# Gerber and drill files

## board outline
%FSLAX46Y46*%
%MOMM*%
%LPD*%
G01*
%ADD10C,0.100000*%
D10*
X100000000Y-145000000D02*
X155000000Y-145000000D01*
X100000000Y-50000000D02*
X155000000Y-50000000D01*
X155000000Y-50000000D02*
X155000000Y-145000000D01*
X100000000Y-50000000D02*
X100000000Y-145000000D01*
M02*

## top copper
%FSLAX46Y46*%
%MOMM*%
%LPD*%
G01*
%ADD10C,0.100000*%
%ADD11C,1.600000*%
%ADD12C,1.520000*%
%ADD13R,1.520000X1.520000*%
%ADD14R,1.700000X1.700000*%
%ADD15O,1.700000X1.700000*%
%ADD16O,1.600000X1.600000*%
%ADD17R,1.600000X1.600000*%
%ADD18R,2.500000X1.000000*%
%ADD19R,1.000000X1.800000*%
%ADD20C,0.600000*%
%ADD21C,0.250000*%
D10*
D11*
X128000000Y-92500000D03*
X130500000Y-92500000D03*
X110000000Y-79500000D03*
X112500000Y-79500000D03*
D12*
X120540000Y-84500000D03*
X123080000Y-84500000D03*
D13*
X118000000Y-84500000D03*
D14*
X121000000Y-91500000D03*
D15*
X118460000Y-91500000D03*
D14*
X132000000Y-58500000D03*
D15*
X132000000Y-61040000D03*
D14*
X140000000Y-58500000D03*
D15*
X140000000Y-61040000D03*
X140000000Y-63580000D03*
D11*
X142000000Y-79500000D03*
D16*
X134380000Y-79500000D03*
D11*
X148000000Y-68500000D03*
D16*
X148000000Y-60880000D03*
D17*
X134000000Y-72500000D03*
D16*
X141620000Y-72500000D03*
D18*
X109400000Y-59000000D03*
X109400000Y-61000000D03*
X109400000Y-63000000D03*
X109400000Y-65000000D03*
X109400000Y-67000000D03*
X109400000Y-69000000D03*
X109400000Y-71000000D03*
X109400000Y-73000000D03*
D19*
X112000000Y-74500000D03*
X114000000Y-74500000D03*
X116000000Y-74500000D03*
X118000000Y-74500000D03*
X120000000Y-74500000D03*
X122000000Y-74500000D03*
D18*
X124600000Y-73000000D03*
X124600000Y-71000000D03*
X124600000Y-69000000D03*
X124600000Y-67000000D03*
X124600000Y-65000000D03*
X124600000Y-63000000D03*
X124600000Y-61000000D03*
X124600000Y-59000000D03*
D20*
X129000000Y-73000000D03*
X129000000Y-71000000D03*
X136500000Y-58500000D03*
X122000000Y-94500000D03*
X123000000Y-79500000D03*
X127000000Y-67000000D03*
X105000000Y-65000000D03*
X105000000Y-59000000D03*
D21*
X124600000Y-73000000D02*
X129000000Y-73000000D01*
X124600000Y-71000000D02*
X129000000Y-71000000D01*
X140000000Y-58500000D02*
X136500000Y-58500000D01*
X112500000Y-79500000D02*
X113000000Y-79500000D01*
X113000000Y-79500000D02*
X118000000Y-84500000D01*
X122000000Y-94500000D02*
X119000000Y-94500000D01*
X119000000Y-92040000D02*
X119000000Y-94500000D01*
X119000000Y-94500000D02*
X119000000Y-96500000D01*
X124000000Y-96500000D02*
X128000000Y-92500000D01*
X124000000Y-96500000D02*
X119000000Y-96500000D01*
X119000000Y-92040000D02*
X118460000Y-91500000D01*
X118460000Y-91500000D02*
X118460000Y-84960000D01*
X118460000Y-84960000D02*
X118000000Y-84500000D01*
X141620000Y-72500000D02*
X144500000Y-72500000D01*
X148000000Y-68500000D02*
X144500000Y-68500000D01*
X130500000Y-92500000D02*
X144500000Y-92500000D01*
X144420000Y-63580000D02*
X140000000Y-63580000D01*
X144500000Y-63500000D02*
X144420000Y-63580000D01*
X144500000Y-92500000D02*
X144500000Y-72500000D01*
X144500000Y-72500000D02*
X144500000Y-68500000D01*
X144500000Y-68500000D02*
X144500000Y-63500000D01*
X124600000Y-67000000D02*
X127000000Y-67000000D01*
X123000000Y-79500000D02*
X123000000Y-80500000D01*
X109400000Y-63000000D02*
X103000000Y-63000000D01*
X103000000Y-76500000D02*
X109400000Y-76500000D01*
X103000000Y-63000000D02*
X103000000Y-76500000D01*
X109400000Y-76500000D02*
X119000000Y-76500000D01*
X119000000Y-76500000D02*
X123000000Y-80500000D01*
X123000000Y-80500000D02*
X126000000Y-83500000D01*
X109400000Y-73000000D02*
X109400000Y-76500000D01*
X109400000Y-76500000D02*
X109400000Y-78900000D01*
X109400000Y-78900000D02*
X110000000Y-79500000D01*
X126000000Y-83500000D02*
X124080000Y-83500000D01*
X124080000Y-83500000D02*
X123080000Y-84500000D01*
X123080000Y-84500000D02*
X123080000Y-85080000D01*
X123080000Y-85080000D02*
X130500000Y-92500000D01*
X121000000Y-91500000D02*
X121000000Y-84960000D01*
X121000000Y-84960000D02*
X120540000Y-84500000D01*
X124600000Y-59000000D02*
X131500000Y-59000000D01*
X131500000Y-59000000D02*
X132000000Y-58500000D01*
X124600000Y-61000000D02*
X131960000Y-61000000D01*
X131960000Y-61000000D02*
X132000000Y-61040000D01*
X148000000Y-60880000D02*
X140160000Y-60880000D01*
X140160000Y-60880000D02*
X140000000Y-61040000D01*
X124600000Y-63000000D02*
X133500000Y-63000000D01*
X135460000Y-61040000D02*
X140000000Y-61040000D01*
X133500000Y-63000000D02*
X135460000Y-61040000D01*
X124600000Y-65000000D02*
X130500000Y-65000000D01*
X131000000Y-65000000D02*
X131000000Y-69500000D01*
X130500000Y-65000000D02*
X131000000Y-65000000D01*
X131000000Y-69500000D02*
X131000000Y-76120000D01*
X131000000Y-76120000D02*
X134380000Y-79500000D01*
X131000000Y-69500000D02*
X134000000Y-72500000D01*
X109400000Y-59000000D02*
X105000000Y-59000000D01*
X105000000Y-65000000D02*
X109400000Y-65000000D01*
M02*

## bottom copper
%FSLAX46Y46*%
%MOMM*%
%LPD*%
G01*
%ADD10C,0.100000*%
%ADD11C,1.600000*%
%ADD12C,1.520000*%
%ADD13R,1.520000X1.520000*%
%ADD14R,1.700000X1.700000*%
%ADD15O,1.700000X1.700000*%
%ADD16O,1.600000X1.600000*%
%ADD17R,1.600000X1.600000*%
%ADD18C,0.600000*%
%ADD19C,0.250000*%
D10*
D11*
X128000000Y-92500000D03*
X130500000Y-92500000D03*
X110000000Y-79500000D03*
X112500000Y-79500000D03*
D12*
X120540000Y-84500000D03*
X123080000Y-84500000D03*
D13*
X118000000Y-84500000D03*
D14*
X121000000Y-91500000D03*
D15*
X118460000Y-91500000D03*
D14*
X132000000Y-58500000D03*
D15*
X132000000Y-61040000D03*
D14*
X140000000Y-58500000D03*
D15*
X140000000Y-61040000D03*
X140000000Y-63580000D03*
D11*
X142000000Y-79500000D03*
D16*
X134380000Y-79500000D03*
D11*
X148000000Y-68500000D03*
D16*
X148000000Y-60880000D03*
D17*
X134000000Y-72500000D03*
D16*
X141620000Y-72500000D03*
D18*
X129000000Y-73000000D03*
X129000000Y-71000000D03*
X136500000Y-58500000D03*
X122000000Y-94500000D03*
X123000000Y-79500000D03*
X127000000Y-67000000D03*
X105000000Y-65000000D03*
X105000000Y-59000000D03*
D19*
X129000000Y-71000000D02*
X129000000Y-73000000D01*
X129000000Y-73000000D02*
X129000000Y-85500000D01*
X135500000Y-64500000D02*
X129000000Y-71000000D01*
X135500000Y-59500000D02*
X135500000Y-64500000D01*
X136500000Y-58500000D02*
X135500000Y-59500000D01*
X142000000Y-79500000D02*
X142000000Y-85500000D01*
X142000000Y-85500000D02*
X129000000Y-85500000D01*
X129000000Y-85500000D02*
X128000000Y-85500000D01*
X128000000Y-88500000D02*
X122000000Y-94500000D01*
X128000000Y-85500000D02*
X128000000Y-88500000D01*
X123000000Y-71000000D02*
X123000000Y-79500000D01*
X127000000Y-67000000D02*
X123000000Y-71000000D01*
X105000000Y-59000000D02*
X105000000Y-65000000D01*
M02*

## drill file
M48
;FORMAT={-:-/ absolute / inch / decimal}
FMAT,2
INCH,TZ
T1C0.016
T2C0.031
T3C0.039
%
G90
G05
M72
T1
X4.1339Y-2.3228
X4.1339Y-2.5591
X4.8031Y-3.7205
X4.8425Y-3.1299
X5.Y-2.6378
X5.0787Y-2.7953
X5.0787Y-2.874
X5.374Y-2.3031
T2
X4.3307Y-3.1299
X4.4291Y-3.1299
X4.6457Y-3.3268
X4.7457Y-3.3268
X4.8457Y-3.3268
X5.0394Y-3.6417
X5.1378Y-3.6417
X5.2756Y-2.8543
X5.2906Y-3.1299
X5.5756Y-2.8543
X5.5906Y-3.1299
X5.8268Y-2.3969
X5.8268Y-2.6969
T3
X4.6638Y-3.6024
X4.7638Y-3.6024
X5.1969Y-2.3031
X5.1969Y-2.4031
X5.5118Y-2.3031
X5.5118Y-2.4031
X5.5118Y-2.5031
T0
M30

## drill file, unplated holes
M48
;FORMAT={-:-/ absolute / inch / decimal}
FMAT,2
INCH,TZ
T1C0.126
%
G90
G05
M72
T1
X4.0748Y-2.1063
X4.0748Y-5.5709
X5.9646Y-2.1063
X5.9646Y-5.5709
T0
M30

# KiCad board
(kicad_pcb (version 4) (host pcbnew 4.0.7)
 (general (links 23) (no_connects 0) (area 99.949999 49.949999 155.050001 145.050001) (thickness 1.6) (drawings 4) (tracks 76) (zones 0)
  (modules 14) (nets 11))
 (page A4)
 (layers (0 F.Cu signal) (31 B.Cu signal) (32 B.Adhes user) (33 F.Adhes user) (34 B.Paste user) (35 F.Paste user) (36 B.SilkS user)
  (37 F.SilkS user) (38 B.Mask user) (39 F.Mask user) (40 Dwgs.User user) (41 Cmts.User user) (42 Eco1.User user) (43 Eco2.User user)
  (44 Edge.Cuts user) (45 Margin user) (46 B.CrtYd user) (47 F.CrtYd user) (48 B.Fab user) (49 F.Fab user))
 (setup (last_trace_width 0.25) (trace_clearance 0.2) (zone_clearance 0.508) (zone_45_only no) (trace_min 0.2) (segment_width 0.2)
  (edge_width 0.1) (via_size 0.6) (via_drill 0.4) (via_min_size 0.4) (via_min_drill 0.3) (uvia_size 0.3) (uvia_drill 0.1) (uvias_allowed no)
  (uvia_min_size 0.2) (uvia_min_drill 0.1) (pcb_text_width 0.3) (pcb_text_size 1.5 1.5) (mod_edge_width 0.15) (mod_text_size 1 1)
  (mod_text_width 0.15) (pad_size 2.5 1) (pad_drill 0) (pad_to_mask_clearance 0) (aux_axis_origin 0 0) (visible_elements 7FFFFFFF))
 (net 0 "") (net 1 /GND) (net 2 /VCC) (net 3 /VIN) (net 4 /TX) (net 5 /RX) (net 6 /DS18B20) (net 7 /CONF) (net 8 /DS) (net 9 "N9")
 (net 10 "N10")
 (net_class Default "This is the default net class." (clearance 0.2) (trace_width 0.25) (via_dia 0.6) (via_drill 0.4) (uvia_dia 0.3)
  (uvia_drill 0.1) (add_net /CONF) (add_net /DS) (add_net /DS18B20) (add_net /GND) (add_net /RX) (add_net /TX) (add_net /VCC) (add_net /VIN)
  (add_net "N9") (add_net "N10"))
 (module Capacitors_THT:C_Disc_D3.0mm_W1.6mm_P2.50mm (layer F.Cu) (at 128 92.5)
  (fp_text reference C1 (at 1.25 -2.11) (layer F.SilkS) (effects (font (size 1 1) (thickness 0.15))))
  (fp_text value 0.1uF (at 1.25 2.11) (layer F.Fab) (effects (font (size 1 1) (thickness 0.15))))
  (pad 1 thru_hole circle (at 0 0) (size 1.6 1.6) (drill 0.8) (layers *.Cu *.Mask) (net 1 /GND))
  (pad 2 thru_hole circle (at 2.5 0) (size 1.6 1.6) (drill 0.8) (layers *.Cu *.Mask) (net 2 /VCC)))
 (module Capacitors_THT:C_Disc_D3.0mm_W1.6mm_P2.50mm (layer F.Cu) (at 110 79.5)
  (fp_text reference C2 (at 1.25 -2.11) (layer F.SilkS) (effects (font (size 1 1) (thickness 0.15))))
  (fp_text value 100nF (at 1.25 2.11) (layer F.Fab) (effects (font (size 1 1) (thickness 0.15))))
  (pad 1 thru_hole circle (at 0 0) (size 1.6 1.6) (drill 0.8) (layers *.Cu *.Mask) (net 2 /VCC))
  (pad 2 thru_hole circle (at 2.5 0) (size 1.6 1.6) (drill 0.8) (layers *.Cu *.Mask) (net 1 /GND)))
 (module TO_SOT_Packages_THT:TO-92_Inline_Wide (layer F.Cu) (at 118 84.5)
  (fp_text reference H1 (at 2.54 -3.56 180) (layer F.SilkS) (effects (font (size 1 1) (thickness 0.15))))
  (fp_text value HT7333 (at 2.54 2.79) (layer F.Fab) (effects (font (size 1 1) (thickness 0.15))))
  (pad 2 thru_hole circle (at 2.54 0 90) (size 1.52 1.52) (drill 0.8) (layers *.Cu *.Mask) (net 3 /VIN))
  (pad 3 thru_hole circle (at 5.08 0 90) (size 1.52 1.52) (drill 0.8) (layers *.Cu *.Mask) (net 2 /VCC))
  (pad 1 thru_hole rect (at 0 0 90) (size 1.52 1.52) (drill 0.8) (layers *.Cu *.Mask) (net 1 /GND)))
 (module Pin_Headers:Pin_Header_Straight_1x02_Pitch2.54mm (layer F.Cu) (at 121 91.5 270)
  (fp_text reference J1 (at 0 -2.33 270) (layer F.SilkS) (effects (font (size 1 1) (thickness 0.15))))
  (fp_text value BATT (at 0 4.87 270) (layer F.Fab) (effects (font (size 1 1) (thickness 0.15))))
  (pad 1 thru_hole rect (at 0 0 270) (size 1.7 1.7) (drill 1) (layers *.Cu *.Mask) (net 3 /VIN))
  (pad 2 thru_hole oval (at 0 2.54 270) (size 1.7 1.7) (drill 1) (layers *.Cu *.Mask) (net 1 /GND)))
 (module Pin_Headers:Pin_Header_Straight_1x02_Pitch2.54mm (layer F.Cu) (at 132 58.5)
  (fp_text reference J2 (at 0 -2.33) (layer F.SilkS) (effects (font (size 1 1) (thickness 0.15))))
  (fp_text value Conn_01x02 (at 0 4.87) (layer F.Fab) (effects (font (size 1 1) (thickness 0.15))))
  (pad 1 thru_hole rect (at 0 0) (size 1.7 1.7) (drill 1) (layers *.Cu *.Mask) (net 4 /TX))
  (pad 2 thru_hole oval (at 0 2.54) (size 1.7 1.7) (drill 1) (layers *.Cu *.Mask) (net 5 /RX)))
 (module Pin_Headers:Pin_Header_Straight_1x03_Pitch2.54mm (layer F.Cu) (at 140 58.5)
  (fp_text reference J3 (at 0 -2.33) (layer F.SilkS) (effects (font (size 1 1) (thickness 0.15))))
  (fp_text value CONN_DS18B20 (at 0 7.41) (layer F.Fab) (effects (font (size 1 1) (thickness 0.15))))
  (pad 1 thru_hole rect (at 0 0) (size 1.7 1.7) (drill 1) (layers *.Cu *.Mask) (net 1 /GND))
  (pad 2 thru_hole oval (at 0 2.54) (size 1.7 1.7) (drill 1) (layers *.Cu *.Mask) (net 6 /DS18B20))
  (pad 3 thru_hole oval (at 0 5.08) (size 1.7 1.7) (drill 1) (layers *.Cu *.Mask) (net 2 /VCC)))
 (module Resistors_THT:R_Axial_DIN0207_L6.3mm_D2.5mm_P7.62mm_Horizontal (layer F.Cu) (at 142 79.5 180)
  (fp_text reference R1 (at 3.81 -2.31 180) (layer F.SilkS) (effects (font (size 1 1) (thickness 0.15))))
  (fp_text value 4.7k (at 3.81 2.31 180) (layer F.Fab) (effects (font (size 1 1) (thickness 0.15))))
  (pad 1 thru_hole circle (at 0 0 180) (size 1.6 1.6) (drill 0.8) (layers *.Cu *.Mask) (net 1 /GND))
  (pad 2 thru_hole oval (at 7.62 0 180) (size 1.6 1.6) (drill 0.8) (layers *.Cu *.Mask) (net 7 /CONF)))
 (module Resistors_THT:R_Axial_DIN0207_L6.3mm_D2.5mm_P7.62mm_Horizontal (layer F.Cu) (at 148 68.5 90)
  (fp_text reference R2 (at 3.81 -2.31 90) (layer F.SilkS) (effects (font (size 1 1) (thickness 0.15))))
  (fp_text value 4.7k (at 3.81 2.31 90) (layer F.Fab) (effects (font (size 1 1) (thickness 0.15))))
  (pad 1 thru_hole circle (at 0 0 90) (size 1.6 1.6) (drill 0.8) (layers *.Cu *.Mask) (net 2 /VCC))
  (pad 2 thru_hole oval (at 7.62 0 90) (size 1.6 1.6) (drill 0.8) (layers *.Cu *.Mask) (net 6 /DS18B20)))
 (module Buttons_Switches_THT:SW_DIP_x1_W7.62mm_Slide (layer F.Cu) (at 134 72.5)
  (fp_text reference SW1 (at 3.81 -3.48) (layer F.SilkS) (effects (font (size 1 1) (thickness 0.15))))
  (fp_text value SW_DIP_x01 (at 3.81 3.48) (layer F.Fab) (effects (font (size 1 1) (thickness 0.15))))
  (pad 1 thru_hole rect (at 0 0) (size 1.6 1.6) (drill 0.8) (layers *.Cu *.Mask) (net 7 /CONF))
  (pad 2 thru_hole oval (at 7.62 0) (size 1.6 1.6) (drill 0.8) (layers *.Cu *.Mask) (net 2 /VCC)))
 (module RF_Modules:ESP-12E (layer F.Cu) (at 117 62.5)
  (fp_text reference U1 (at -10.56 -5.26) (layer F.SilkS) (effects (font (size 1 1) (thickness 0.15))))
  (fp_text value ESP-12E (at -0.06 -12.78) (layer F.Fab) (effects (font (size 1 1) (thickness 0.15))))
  (pad 1 smd rect (at -7.6 -3.5) (size 2.5 1) (layers F.Cu F.Paste F.Mask) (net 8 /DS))
  (pad 2 smd rect (at -7.6 -1.5) (size 2.5 1) (layers F.Cu F.Paste F.Mask))
  (pad 3 smd rect (at -7.6 0.5) (size 2.5 1) (layers F.Cu F.Paste F.Mask) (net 2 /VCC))
  (pad 4 smd rect (at -7.6 2.5) (size 2.5 1) (layers F.Cu F.Paste F.Mask) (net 8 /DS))
  (pad 5 smd rect (at -7.6 4.5) (size 2.5 1) (layers F.Cu F.Paste F.Mask))
  (pad 6 smd rect (at -7.6 6.5) (size 2.5 1) (layers F.Cu F.Paste F.Mask))
  (pad 7 smd rect (at -7.6 8.5) (size 2.5 1) (layers F.Cu F.Paste F.Mask))
  (pad 8 smd rect (at -7.6 10.5) (size 2.5 1) (layers F.Cu F.Paste F.Mask) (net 2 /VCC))
  (pad 9 smd rect (at -5 12) (size 1 1.8) (layers F.Cu F.Paste F.Mask))
  (pad 10 smd rect (at -3 12) (size 1 1.8) (layers F.Cu F.Paste F.Mask))
  (pad 11 smd rect (at -1 12) (size 1 1.8) (layers F.Cu F.Paste F.Mask) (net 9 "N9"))
  (pad 12 smd rect (at 1 12) (size 1 1.8) (layers F.Cu F.Paste F.Mask) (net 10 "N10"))
  (pad 13 smd rect (at 3 12) (size 1 1.8) (layers F.Cu F.Paste F.Mask))
  (pad 14 smd rect (at 5 12) (size 1 1.8) (layers F.Cu F.Paste F.Mask))
  (pad 15 smd rect (at 7.6 10.5) (size 2.5 1) (layers F.Cu F.Paste F.Mask) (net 1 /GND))
  (pad 16 smd rect (at 7.6 8.5) (size 2.5 1) (layers F.Cu F.Paste F.Mask) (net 1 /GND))
  (pad 17 smd rect (at 7.6 6.5) (size 2.5 1) (layers F.Cu F.Paste F.Mask))
  (pad 18 smd rect (at 7.6 4.5) (size 2.5 1) (layers F.Cu F.Paste F.Mask) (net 2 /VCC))
  (pad 19 smd rect (at 7.6 2.5) (size 2.5 1) (layers F.Cu F.Paste F.Mask) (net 7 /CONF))
  (pad 20 smd rect (at 7.6 0.5) (size 2.5 1) (layers F.Cu F.Paste F.Mask) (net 6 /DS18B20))
  (pad 21 smd rect (at 7.6 -1.5) (size 2.5 1) (layers F.Cu F.Paste F.Mask) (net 5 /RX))
  (pad 22 smd rect (at 7.6 -3.5) (size 2.5 1) (layers F.Cu F.Paste F.Mask) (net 4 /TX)))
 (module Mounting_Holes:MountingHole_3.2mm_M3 (layer F.Cu) (at 103.5 53.5)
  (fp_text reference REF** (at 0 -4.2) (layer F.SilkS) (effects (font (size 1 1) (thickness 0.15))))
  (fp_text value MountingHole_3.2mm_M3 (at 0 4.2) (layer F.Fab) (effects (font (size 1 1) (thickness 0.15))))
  (pad 1 np_thru_hole circle (at 0 0) (size 3.2 3.2) (drill 3.2) (layers *.Cu *.Mask)))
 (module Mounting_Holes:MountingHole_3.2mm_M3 (layer F.Cu) (at 151.5 53.5)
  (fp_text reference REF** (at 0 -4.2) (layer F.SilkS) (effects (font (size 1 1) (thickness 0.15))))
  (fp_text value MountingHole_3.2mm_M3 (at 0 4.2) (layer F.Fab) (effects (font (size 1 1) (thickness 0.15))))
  (pad 1 np_thru_hole circle (at 0 0) (size 3.2 3.2) (drill 3.2) (layers *.Cu *.Mask)))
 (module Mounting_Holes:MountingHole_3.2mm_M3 (layer F.Cu) (at 151.5 141.5)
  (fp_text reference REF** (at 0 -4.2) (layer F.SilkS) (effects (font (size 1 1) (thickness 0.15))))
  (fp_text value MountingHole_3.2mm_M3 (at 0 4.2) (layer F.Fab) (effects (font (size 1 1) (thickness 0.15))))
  (pad 1 np_thru_hole circle (at 0 0) (size 3.2 3.2) (drill 3.2) (layers *.Cu *.Mask)))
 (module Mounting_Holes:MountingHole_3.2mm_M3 (layer F.Cu) (at 103.5 141.5)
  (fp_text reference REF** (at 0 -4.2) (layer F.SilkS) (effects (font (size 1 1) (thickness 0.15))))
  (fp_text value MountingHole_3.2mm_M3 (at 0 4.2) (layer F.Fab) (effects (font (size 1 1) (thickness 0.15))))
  (pad 1 np_thru_hole circle (at 0 0) (size 3.2 3.2) (drill 3.2) (layers *.Cu *.Mask)))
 (gr_line (start 100 145) (end 155 145) (angle 90) (layer Edge.Cuts) (width 0.1))
 (gr_line (start 100 50) (end 155 50) (angle 90) (layer Edge.Cuts) (width 0.1))
 (gr_line (start 155 50) (end 155 145) (angle 90) (layer Edge.Cuts) (width 0.1))
 (gr_line (start 100 50) (end 100 145) (angle 90) (layer Edge.Cuts) (width 0.1))
 (segment (start 124.6 73) (end 129 73) (width 0.25) (layer F.Cu) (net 1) (status 400000))
 (via (at 129 73) (size 0.6) (drill 0.4) (layers F.Cu B.Cu) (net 1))
 (segment (start 124.6 71) (end 129 71) (width 0.25) (layer F.Cu) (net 1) (status 400000))
 (via (at 129 71) (size 0.6) (drill 0.4) (layers F.Cu B.Cu) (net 1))
 (segment (start 140 58.5) (end 136.5 58.5) (width 0.25) (layer F.Cu) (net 1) (status 400000))
 (segment (start 129 71) (end 129 73) (width 0.25) (layer B.Cu) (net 1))
 (segment (start 129 73) (end 129 85.5) (width 0.25) (layer B.Cu) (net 1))
 (segment (start 135.5 64.5) (end 129 71) (width 0.25) (layer B.Cu) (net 1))
 (segment (start 135.5 59.5) (end 135.5 64.5) (width 0.25) (layer B.Cu) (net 1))
 (segment (start 136.5 58.5) (end 135.5 59.5) (width 0.25) (layer B.Cu) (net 1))
 (via (at 136.5 58.5) (size 0.6) (drill 0.4) (layers F.Cu B.Cu) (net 1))
 (segment (start 142 79.5) (end 142 85.5) (width 0.25) (layer B.Cu) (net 1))
 (segment (start 142 85.5) (end 129 85.5) (width 0.25) (layer B.Cu) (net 1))
 (segment (start 129 85.5) (end 128 85.5) (width 0.25) (layer B.Cu) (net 1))
 (segment (start 112.5 79.5) (end 113 79.5) (width 0.25) (layer F.Cu) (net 1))
 (segment (start 113 79.5) (end 118 84.5) (width 0.25) (layer F.Cu) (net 1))
 (segment (start 128 88.5) (end 122 94.5) (width 0.25) (layer B.Cu) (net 1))
 (segment (start 128 85.5) (end 128 88.5) (width 0.25) (layer B.Cu) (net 1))
 (segment (start 122 94.5) (end 119 94.5) (width 0.25) (layer F.Cu) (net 1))
 (via (at 122 94.5) (size 0.6) (drill 0.4) (layers F.Cu B.Cu) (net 1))
 (segment (start 119 92.04) (end 119 94.5) (width 0.25) (layer F.Cu) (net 1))
 (segment (start 119 94.5) (end 119 96.5) (width 0.25) (layer F.Cu) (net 1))
 (segment (start 124 96.5) (end 128 92.5) (width 0.25) (layer F.Cu) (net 1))
 (segment (start 124 96.5) (end 119 96.5) (width 0.25) (layer F.Cu) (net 1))
 (segment (start 119 92.04) (end 118.46 91.5) (width 0.25) (layer F.Cu) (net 1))
 (segment (start 118.46 91.5) (end 118.46 84.96) (width 0.25) (layer F.Cu) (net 1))
 (segment (start 118.46 84.96) (end 118 84.5) (width 0.25) (layer F.Cu) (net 1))
 (segment (start 141.62 72.5) (end 144.5 72.5) (width 0.25) (layer F.Cu) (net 2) (status 400000))
 (segment (start 148 68.5) (end 144.5 68.5) (width 0.25) (layer F.Cu) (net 2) (status 400000))
 (segment (start 130.5 92.5) (end 144.5 92.5) (width 0.25) (layer F.Cu) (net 2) (status 400000))
 (segment (start 144.42 63.58) (end 140 63.58) (width 0.25) (layer F.Cu) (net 2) (status 800000))
 (segment (start 144.5 63.5) (end 144.42 63.58) (width 0.25) (layer F.Cu) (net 2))
 (segment (start 144.5 92.5) (end 144.5 72.5) (width 0.25) (layer F.Cu) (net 2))
 (segment (start 144.5 72.5) (end 144.5 68.5) (width 0.25) (layer F.Cu) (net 2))
 (segment (start 144.5 68.5) (end 144.5 63.5) (width 0.25) (layer F.Cu) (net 2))
 (segment (start 124.6 67) (end 127 67) (width 0.25) (layer F.Cu) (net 2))
 (segment (start 123 79.5) (end 123 80.5) (width 0.25) (layer F.Cu) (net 2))
 (via (at 123 79.5) (size 0.6) (drill 0.4) (layers F.Cu B.Cu) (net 2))
 (segment (start 123 71) (end 123 79.5) (width 0.25) (layer B.Cu) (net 2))
 (segment (start 127 67) (end 123 71) (width 0.25) (layer B.Cu) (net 2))
 (via (at 127 67) (size 0.6) (drill 0.4) (layers F.Cu B.Cu) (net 2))
 (segment (start 109.4 63) (end 103 63) (width 0.25) (layer F.Cu) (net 2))
 (segment (start 103 76.5) (end 109.4 76.5) (width 0.25) (layer F.Cu) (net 2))
 (segment (start 103 63) (end 103 76.5) (width 0.25) (layer F.Cu) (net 2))
 (segment (start 109.4 76.5) (end 119 76.5) (width 0.25) (layer F.Cu) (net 2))
 (segment (start 119 76.5) (end 123 80.5) (width 0.25) (layer F.Cu) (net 2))
 (segment (start 123 80.5) (end 126 83.5) (width 0.25) (layer F.Cu) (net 2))
 (segment (start 109.4 73) (end 109.4 76.5) (width 0.25) (layer F.Cu) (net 2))
 (segment (start 109.4 76.5) (end 109.4 78.9) (width 0.25) (layer F.Cu) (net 2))
 (segment (start 109.4 78.9) (end 110 79.5) (width 0.25) (layer F.Cu) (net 2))
 (segment (start 126 83.5) (end 124.08 83.5) (width 0.25) (layer F.Cu) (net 2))
 (segment (start 124.08 83.5) (end 123.08 84.5) (width 0.25) (layer F.Cu) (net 2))
 (segment (start 123.08 84.5) (end 123.08 85.08) (width 0.25) (layer F.Cu) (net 2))
 (segment (start 123.08 85.08) (end 130.5 92.5) (width 0.25) (layer F.Cu) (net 2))
 (segment (start 121 91.5) (end 121 84.96) (width 0.25) (layer F.Cu) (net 3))
 (segment (start 121 84.96) (end 120.54 84.5) (width 0.25) (layer F.Cu) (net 3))
 (segment (start 124.6 59) (end 131.5 59) (width 0.25) (layer F.Cu) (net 4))
 (segment (start 131.5 59) (end 132 58.5) (width 0.25) (layer F.Cu) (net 4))
 (segment (start 124.6 61) (end 131.96 61) (width 0.25) (layer F.Cu) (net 5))
 (segment (start 131.96 61) (end 132 61.04) (width 0.25) (layer F.Cu) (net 5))
 (segment (start 148 60.88) (end 140.16 60.88) (width 0.25) (layer F.Cu) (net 6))
 (segment (start 140.16 60.88) (end 140 61.04) (width 0.25) (layer F.Cu) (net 6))
 (segment (start 124.6 63) (end 133.5 63) (width 0.25) (layer F.Cu) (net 6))
 (segment (start 135.46 61.04) (end 140 61.04) (width 0.25) (layer F.Cu) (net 6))
 (segment (start 133.5 63) (end 135.46 61.04) (width 0.25) (layer F.Cu) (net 6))
 (segment (start 124.6 65) (end 130.5 65) (width 0.25) (layer F.Cu) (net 7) (status 400000))
 (segment (start 131 65) (end 131 69.5) (width 0.25) (layer F.Cu) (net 7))
 (segment (start 130.5 65) (end 131 65) (width 0.25) (layer F.Cu) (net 7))
 (segment (start 131 69.5) (end 131 76.12) (width 0.25) (layer F.Cu) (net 7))
 (segment (start 131 76.12) (end 134.38 79.5) (width 0.25) (layer F.Cu) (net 7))
 (segment (start 131 69.5) (end 134 72.5) (width 0.25) (layer F.Cu) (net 7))
 (segment (start 109.4 59) (end 105 59) (width 0.25) (layer F.Cu) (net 8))
 (segment (start 105 65) (end 109.4 65) (width 0.25) (layer F.Cu) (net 8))
 (via (at 105 65) (size 0.6) (drill 0.4) (layers F.Cu B.Cu) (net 8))
 (segment (start 105 59) (end 105 65) (width 0.25) (layer B.Cu) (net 8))
 (via (at 105 59) (size 0.6) (drill 0.4) (layers F.Cu B.Cu) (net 8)))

